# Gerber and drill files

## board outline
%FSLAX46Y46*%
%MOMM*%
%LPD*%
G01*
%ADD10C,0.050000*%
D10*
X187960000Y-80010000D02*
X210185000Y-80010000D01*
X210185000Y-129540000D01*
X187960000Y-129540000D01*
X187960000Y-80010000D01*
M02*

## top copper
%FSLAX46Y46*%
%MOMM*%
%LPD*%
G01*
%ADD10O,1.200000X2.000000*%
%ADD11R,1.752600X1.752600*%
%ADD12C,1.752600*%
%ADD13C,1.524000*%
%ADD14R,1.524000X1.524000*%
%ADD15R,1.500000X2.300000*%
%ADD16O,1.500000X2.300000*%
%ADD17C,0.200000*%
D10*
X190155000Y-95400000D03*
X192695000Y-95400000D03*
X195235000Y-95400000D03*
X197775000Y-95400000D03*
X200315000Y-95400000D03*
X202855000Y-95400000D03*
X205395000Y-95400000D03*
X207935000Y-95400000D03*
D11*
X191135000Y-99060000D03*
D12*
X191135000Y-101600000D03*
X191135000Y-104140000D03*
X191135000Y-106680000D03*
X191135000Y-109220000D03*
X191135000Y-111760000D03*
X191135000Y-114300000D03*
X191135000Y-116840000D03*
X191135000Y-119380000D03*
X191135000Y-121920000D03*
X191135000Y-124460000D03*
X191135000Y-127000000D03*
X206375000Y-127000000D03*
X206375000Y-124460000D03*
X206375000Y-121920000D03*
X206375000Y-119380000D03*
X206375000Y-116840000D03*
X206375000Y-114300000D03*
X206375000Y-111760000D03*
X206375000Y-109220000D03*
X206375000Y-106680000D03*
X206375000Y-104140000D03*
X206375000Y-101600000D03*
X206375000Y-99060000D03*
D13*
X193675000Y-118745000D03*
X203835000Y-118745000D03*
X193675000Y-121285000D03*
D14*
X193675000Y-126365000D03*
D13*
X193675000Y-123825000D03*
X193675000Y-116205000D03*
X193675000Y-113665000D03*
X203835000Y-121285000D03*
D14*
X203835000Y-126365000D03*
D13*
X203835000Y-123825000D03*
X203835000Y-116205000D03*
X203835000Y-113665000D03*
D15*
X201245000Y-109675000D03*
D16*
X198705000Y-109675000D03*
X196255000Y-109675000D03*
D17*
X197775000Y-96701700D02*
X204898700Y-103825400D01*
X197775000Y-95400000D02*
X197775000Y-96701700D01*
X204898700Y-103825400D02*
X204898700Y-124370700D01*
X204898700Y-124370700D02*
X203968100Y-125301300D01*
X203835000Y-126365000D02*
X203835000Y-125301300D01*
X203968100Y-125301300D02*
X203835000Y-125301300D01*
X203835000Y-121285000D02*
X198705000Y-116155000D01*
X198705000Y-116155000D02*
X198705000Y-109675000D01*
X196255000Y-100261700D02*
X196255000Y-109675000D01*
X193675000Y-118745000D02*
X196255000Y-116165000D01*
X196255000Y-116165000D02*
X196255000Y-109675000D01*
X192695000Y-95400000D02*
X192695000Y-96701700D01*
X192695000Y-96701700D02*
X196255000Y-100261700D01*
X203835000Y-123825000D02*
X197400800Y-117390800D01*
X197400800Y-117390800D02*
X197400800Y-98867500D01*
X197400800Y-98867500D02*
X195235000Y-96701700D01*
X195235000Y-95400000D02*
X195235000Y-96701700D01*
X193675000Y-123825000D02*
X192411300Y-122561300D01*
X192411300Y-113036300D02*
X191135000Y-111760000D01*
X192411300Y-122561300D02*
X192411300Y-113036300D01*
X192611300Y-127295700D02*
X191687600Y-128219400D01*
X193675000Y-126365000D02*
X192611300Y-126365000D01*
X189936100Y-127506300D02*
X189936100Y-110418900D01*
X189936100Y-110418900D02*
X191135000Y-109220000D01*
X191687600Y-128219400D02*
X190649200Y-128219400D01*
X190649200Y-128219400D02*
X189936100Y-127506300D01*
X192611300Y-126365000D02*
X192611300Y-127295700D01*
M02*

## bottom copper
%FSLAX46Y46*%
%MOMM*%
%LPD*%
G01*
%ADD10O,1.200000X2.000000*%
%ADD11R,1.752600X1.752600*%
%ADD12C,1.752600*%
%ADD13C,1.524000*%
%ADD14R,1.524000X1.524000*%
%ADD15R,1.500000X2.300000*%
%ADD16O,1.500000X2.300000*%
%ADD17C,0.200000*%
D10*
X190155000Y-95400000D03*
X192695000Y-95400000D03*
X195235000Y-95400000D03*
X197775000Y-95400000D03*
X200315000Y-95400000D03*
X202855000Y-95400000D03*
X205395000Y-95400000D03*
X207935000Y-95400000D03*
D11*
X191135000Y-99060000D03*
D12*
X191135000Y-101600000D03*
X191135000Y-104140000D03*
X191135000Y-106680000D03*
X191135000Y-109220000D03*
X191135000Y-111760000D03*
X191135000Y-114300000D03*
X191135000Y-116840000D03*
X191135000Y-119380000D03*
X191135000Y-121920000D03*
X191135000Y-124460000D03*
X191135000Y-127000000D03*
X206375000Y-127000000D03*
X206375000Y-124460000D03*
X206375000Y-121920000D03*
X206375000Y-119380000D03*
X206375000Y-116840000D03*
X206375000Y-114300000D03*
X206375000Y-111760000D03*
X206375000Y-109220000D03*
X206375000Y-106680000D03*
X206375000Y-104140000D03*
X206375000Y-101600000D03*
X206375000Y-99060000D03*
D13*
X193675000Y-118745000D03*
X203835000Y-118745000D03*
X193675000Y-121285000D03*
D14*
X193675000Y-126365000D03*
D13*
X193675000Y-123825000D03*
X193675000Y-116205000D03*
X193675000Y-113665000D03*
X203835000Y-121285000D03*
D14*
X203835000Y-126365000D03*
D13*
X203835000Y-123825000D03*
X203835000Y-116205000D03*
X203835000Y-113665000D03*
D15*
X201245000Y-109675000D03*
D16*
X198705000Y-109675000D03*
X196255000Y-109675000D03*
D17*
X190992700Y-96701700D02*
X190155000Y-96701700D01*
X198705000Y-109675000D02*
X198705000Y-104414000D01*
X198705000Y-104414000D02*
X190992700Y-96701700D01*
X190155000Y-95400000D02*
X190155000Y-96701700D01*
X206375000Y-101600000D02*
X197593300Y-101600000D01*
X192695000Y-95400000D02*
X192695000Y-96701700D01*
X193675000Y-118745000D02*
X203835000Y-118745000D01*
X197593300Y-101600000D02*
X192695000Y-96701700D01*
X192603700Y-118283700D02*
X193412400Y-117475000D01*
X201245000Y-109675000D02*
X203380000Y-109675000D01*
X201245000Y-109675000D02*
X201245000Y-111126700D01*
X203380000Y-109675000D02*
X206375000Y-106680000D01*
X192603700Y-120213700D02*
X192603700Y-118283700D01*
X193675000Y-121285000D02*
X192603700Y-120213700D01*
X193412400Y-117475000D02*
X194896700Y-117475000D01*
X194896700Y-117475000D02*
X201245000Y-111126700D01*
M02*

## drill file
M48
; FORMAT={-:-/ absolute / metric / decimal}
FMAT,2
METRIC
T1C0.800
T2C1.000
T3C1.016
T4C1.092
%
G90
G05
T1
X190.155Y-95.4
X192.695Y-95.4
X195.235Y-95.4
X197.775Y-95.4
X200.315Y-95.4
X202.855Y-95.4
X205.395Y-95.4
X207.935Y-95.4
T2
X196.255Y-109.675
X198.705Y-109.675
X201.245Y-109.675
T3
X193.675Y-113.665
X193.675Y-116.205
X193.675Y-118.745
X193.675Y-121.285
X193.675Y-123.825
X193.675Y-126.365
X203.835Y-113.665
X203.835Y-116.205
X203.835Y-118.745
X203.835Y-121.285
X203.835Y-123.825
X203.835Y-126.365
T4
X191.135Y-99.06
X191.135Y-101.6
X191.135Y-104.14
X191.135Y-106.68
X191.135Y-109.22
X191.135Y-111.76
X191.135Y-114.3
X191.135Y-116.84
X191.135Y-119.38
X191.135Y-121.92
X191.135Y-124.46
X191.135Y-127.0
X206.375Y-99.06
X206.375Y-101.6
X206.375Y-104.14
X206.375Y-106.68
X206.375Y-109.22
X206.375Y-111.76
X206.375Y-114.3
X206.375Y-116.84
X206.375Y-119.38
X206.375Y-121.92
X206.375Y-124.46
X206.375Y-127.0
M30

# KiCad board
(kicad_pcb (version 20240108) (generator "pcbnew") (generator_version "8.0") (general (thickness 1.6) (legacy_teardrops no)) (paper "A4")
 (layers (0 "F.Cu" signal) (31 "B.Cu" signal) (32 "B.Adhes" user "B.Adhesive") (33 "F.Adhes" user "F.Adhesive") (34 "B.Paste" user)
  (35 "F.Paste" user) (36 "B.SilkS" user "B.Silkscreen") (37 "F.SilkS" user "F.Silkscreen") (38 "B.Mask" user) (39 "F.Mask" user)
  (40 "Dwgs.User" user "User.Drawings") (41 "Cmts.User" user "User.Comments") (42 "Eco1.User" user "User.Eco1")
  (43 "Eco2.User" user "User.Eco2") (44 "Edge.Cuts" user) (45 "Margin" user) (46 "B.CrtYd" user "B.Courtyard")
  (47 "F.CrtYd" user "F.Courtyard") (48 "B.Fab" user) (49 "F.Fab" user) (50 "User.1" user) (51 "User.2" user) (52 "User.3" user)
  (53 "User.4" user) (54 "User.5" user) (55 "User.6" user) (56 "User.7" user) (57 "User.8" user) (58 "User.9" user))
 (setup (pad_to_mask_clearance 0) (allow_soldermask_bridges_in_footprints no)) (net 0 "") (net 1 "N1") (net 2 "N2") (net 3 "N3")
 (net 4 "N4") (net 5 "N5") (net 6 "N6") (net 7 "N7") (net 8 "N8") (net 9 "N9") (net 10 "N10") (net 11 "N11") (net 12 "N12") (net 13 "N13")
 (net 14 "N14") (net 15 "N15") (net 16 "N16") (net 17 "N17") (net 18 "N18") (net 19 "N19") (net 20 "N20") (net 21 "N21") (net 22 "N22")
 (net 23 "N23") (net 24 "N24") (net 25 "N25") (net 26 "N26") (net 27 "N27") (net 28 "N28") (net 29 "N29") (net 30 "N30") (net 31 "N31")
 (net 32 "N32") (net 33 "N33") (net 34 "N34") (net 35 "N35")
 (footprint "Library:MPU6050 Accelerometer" (layer "F.Cu") (at 201.295 88.9 90)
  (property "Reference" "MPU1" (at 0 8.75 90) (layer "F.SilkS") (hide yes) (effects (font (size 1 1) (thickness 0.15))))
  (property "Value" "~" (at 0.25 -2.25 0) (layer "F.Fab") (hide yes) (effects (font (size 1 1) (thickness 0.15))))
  (pad "1" thru_hole oval (at -6.5 -11.14) (size 1.2 2) (drill 0.8) (layers "*.Cu" "*.Mask") (remove_unused_layers no) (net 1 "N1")
   (thermal_bridge_angle 45))
  (pad "2" thru_hole oval (at -6.5 -8.6) (size 1.2 2) (drill 0.8) (layers "*.Cu" "*.Mask") (remove_unused_layers no) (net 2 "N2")
   (thermal_bridge_angle 45))
  (pad "3" thru_hole oval (at -6.5 -6.06) (size 1.2 2) (drill 0.8) (layers "*.Cu" "*.Mask") (remove_unused_layers no) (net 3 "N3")
   (thermal_bridge_angle 45))
  (pad "4" thru_hole oval (at -6.5 -3.52) (size 1.2 2) (drill 0.8) (layers "*.Cu" "*.Mask") (remove_unused_layers no) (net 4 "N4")
   (thermal_bridge_angle 45))
  (pad "5" thru_hole oval (at -6.5 -0.98) (size 1.2 2) (drill 0.8) (layers "*.Cu" "*.Mask") (remove_unused_layers no) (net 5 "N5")
   (thermal_bridge_angle 45))
  (pad "6" thru_hole oval (at -6.5 1.56) (size 1.2 2) (drill 0.8) (layers "*.Cu" "*.Mask") (remove_unused_layers no) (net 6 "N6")
   (thermal_bridge_angle 45))
  (pad "7" thru_hole oval (at -6.5 4.1) (size 1.2 2) (drill 0.8) (layers "*.Cu" "*.Mask") (remove_unused_layers no) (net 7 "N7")
   (thermal_bridge_angle 45))
  (pad "8" thru_hole oval (at -6.5 6.64) (size 1.2 2) (drill 0.8) (layers "*.Cu" "*.Mask") (remove_unused_layers no) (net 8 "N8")
   (thermal_bridge_angle 45)))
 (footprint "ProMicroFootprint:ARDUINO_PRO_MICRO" (layer "F.Cu") (at 198.755 113.03 -90)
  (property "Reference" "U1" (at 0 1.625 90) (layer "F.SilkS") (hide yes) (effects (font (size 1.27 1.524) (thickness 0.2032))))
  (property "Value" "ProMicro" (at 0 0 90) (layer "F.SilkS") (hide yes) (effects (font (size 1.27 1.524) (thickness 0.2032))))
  (pad "1" thru_hole rect (at -13.97 7.62 270) (size 1.7526 1.7526) (drill 1.0922) (layers "*.Cu" "*.SilkS" "*.Mask")
   (remove_unused_layers no) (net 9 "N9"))
  (pad "2" thru_hole circle (at -11.43 7.62 270) (size 1.7526 1.7526) (drill 1.0922) (layers "*.Cu" "*.SilkS" "*.Mask")
   (remove_unused_layers no) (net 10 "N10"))
  (pad "3" thru_hole circle (at -8.89 7.62 270) (size 1.7526 1.7526) (drill 1.0922) (layers "*.Cu" "*.SilkS" "*.Mask")
   (remove_unused_layers no) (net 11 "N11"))
  (pad "4" thru_hole circle (at -6.35 7.62 270) (size 1.7526 1.7526) (drill 1.0922) (layers "*.Cu" "*.SilkS" "*.Mask")
   (remove_unused_layers no) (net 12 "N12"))
  (pad "5" thru_hole circle (at -3.81 7.62 270) (size 1.7526 1.7526) (drill 1.0922) (layers "*.Cu" "*.SilkS" "*.Mask")
   (remove_unused_layers no) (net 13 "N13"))
  (pad "6" thru_hole circle (at -1.27 7.62 270) (size 1.7526 1.7526) (drill 1.0922) (layers "*.Cu" "*.SilkS" "*.Mask")
   (remove_unused_layers no) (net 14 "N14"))
  (pad "7" thru_hole circle (at 1.27 7.62 270) (size 1.7526 1.7526) (drill 1.0922) (layers "*.Cu" "*.SilkS" "*.Mask")
   (remove_unused_layers no) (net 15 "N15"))
  (pad "8" thru_hole circle (at 3.81 7.62 270) (size 1.7526 1.7526) (drill 1.0922) (layers "*.Cu" "*.SilkS" "*.Mask")
   (remove_unused_layers no) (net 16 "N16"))
  (pad "9" thru_hole circle (at 6.35 7.62 270) (size 1.7526 1.7526) (drill 1.0922) (layers "*.Cu" "*.SilkS" "*.Mask")
   (remove_unused_layers no) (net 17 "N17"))
  (pad "10" thru_hole circle (at 8.89 7.62 270) (size 1.7526 1.7526) (drill 1.0922) (layers "*.Cu" "*.SilkS" "*.Mask")
   (remove_unused_layers no) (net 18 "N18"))
  (pad "11" thru_hole circle (at 11.43 7.62 270) (size 1.7526 1.7526) (drill 1.0922) (layers "*.Cu" "*.SilkS" "*.Mask")
   (remove_unused_layers no) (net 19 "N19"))
  (pad "12" thru_hole circle (at 13.97 7.62 270) (size 1.7526 1.7526) (drill 1.0922) (layers "*.Cu" "*.SilkS" "*.Mask")
   (remove_unused_layers no) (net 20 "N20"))
  (pad "13" thru_hole circle (at 13.97 -7.62 270) (size 1.7526 1.7526) (drill 1.0922) (layers "*.Cu" "*.SilkS" "*.Mask")
   (remove_unused_layers no) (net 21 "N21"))
  (pad "14" thru_hole circle (at 11.43 -7.62 270) (size 1.7526 1.7526) (drill 1.0922) (layers "*.Cu" "*.SilkS" "*.Mask")
   (remove_unused_layers no) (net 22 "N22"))
  (pad "15" thru_hole circle (at 8.89 -7.62 270) (size 1.7526 1.7526) (drill 1.0922) (layers "*.Cu" "*.SilkS" "*.Mask")
   (remove_unused_layers no) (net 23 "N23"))
  (pad "16" thru_hole circle (at 6.35 -7.62 270) (size 1.7526 1.7526) (drill 1.0922) (layers "*.Cu" "*.SilkS" "*.Mask")
   (remove_unused_layers no) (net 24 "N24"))
  (pad "17" thru_hole circle (at 3.81 -7.62 270) (size 1.7526 1.7526) (drill 1.0922) (layers "*.Cu" "*.SilkS" "*.Mask")
   (remove_unused_layers no) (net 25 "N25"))
  (pad "18" thru_hole circle (at 1.27 -7.62 270) (size 1.7526 1.7526) (drill 1.0922) (layers "*.Cu" "*.SilkS" "*.Mask")
   (remove_unused_layers no) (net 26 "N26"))
  (pad "19" thru_hole circle (at -1.27 -7.62 270) (size 1.7526 1.7526) (drill 1.0922) (layers "*.Cu" "*.SilkS" "*.Mask")
   (remove_unused_layers no) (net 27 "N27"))
  (pad "20" thru_hole circle (at -3.81 -7.62 270) (size 1.7526 1.7526) (drill 1.0922) (layers "*.Cu" "*.SilkS" "*.Mask")
   (remove_unused_layers no) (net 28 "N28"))
  (pad "21" thru_hole circle (at -6.35 -7.62 270) (size 1.7526 1.7526) (drill 1.0922) (layers "*.Cu" "*.SilkS" "*.Mask")
   (remove_unused_layers no) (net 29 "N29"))
  (pad "22" thru_hole circle (at -8.89 -7.62 270) (size 1.7526 1.7526) (drill 1.0922) (layers "*.Cu" "*.SilkS" "*.Mask")
   (remove_unused_layers no) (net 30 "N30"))
  (pad "23" thru_hole circle (at -11.43 -7.62 270) (size 1.7526 1.7526) (drill 1.0922) (layers "*.Cu" "*.SilkS" "*.Mask")
   (remove_unused_layers no) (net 2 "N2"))
  (pad "24" thru_hole circle (at -13.97 -7.62 270) (size 1.7526 1.7526) (drill 1.0922) (layers "*.Cu" "*.SilkS" "*.Mask")
   (remove_unused_layers no) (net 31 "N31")))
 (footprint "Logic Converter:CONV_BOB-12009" (layer "F.Cu") (at 198.755 120.015 180)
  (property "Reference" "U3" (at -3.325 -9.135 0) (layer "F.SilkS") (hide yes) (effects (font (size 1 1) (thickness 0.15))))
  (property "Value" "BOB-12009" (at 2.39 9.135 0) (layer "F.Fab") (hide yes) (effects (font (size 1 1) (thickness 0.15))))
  (pad "GND_1" thru_hole circle (at 5.08 1.27 180) (size 1.524 1.524) (drill 1.016) (layers "*.Cu" "*.Mask") (remove_unused_layers no)
   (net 2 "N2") (solder_mask_margin 0.102))
  (pad "GND_2" thru_hole circle (at -5.08 1.27 180) (size 1.524 1.524) (drill 1.016) (layers "*.Cu" "*.Mask") (remove_unused_layers no)
   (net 2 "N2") (solder_mask_margin 0.102))
  (pad "HV" thru_hole circle (at 5.08 -1.27 180) (size 1.524 1.524) (drill 1.016) (layers "*.Cu" "*.Mask") (remove_unused_layers no)
   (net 29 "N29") (solder_mask_margin 0.102))
  (pad "HV1" thru_hole rect (at 5.08 -6.35 180) (size 1.524 1.524) (drill 1.016) (layers "*.Cu" "*.Mask") (remove_unused_layers no)
   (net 13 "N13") (solder_mask_margin 0.102))
  (pad "HV2" thru_hole circle (at 5.08 -3.81 180) (size 1.524 1.524) (drill 1.016) (layers "*.Cu" "*.Mask") (remove_unused_layers no)
   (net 14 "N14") (solder_mask_margin 0.102))
  (pad "HV3" thru_hole circle (at 5.08 3.81 180) (size 1.524 1.524) (drill 1.016) (layers "*.Cu" "*.Mask") (remove_unused_layers no)
   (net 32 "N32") (solder_mask_margin 0.102))
  (pad "HV4" thru_hole circle (at 5.08 6.35 180) (size 1.524 1.524) (drill 1.016) (layers "*.Cu" "*.Mask") (remove_unused_layers no)
   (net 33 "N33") (solder_mask_margin 0.102))
  (pad "LV" thru_hole circle (at -5.08 -1.27 180) (size 1.524 1.524) (drill 1.016) (layers "*.Cu" "*.Mask") (remove_unused_layers no)
   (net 1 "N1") (solder_mask_margin 0.102))
  (pad "LV1" thru_hole rect (at -5.08 -6.35 180) (size 1.524 1.524) (drill 1.016) (layers "*.Cu" "*.Mask") (remove_unused_layers no)
   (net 4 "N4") (solder_mask_margin 0.102))
  (pad "LV2" thru_hole circle (at -5.08 -3.81 180) (size 1.524 1.524) (drill 1.016) (layers "*.Cu" "*.Mask") (remove_unused_layers no)
   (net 3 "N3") (solder_mask_margin 0.102))
  (pad "LV3" thru_hole circle (at -5.08 3.81 180) (size 1.524 1.524) (drill 1.016) (layers "*.Cu" "*.Mask") (remove_unused_layers no)
   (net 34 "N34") (solder_mask_margin 0.102))
  (pad "LV4" thru_hole circle (at -5.08 6.35 180) (size 1.524 1.524) (drill 1.016) (layers "*.Cu" "*.Mask") (remove_unused_layers no)
   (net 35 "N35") (solder_mask_margin 0.102)))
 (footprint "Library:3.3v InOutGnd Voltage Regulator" (layer "F.Cu") (at 198.755 111.175)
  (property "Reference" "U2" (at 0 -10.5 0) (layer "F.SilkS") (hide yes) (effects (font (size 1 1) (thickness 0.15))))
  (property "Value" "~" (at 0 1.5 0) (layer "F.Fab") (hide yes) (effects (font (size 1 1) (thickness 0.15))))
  (pad "1" thru_hole rect (at 2.49 -1.5) (size 1.5 2.3) (drill 1) (layers "*.Cu" "*.Mask") (remove_unused_layers no) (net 29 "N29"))
  (pad "2" thru_hole oval (at -0.05 -1.5) (size 1.5 2.3) (drill 1) (layers "*.Cu" "*.Mask") (remove_unused_layers no) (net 1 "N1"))
  (pad "3" thru_hole oval (at -2.5 -1.5) (size 1.5 2.3) (drill 1) (layers "*.Cu" "*.Mask") (remove_unused_layers no) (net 2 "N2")))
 (gr_rect (start 187.96 80.01) (end 210.185 129.54) (stroke (width 0.05) (type default)) (fill none) (layer "Edge.Cuts"))
 (segment (start 197.775 96.7017) (end 204.8987 103.8254) (width 0.2) (layer "F.Cu") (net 4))
 (segment (start 197.775 95.4) (end 197.775 96.7017) (width 0.2) (layer "F.Cu") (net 4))
 (segment (start 204.8987 103.8254) (end 204.8987 124.3707) (width 0.2) (layer "F.Cu") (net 4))
 (segment (start 204.8987 124.3707) (end 203.9681 125.3013) (width 0.2) (layer "F.Cu") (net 4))
 (segment (start 203.835 126.365) (end 203.835 125.3013) (width 0.2) (layer "F.Cu") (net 4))
 (segment (start 203.9681 125.3013) (end 203.835 125.3013) (width 0.2) (layer "F.Cu") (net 4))
 (segment (start 203.835 121.285) (end 198.705 116.155) (width 0.2) (layer "F.Cu") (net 1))
 (segment (start 198.705 116.155) (end 198.705 109.675) (width 0.2) (layer "F.Cu") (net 1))
 (segment (start 190.9927 96.7017) (end 190.155 96.7017) (width 0.2) (layer "B.Cu") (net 1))
 (segment (start 198.705 109.675) (end 198.705 104.414) (width 0.2) (layer "B.Cu") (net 1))
 (segment (start 198.705 104.414) (end 190.9927 96.7017) (width 0.2) (layer "B.Cu") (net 1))
 (segment (start 190.155 95.4) (end 190.155 96.7017) (width 0.2) (layer "B.Cu") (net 1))
 (segment (start 196.255 100.2617) (end 196.255 109.675) (width 0.2) (layer "F.Cu") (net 2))
 (segment (start 193.675 118.745) (end 196.255 116.165) (width 0.2) (layer "F.Cu") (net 2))
 (segment (start 196.255 116.165) (end 196.255 109.675) (width 0.2) (layer "F.Cu") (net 2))
 (segment (start 192.695 95.4) (end 192.695 96.7017) (width 0.2) (layer "F.Cu") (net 2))
 (segment (start 192.695 96.7017) (end 196.255 100.2617) (width 0.2) (layer "F.Cu") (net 2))
 (segment (start 206.375 101.6) (end 197.5933 101.6) (width 0.2) (layer "B.Cu") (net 2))
 (segment (start 192.695 95.4) (end 192.695 96.7017) (width 0.2) (layer "B.Cu") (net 2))
 (segment (start 193.675 118.745) (end 203.835 118.745) (width 0.2) (layer "B.Cu") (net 2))
 (segment (start 197.5933 101.6) (end 192.695 96.7017) (width 0.2) (layer "B.Cu") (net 2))
 (segment (start 203.835 123.825) (end 197.4008 117.3908) (width 0.2) (layer "F.Cu") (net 3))
 (segment (start 197.4008 117.3908) (end 197.4008 98.8675) (width 0.2) (layer "F.Cu") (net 3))
 (segment (start 197.4008 98.8675) (end 195.235 96.7017) (width 0.2) (layer "F.Cu") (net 3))
 (segment (start 195.235 95.4) (end 195.235 96.7017) (width 0.2) (layer "F.Cu") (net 3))
 (segment (start 192.6037 118.2837) (end 193.4124 117.475) (width 0.2) (layer "B.Cu") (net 29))
 (segment (start 201.245 109.675) (end 203.38 109.675) (width 0.2) (layer "B.Cu") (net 29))
 (segment (start 201.245 109.675) (end 201.245 111.1267) (width 0.2) (layer "B.Cu") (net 29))
 (segment (start 203.38 109.675) (end 206.375 106.68) (width 0.2) (layer "B.Cu") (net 29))
 (segment (start 192.6037 120.2137) (end 192.6037 118.2837) (width 0.2) (layer "B.Cu") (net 29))
 (segment (start 193.675 121.285) (end 192.6037 120.2137) (width 0.2) (layer "B.Cu") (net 29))
 (segment (start 193.4124 117.475) (end 194.8967 117.475) (width 0.2) (layer "B.Cu") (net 29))
 (segment (start 194.8967 117.475) (end 201.245 111.1267) (width 0.2) (layer "B.Cu") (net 29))
 (segment (start 193.675 123.825) (end 192.4113 122.5613) (width 0.2) (layer "F.Cu") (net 14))
 (segment (start 192.4113 113.0363) (end 191.135 111.76) (width 0.2) (layer "F.Cu") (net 14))
 (segment (start 192.4113 122.5613) (end 192.4113 113.0363) (width 0.2) (layer "F.Cu") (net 14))
 (segment (start 192.6113 127.2957) (end 191.6876 128.2194) (width 0.2) (layer "F.Cu") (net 13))
 (segment (start 193.675 126.365) (end 192.6113 126.365) (width 0.2) (layer "F.Cu") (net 13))
 (segment (start 189.9361 127.5063) (end 189.9361 110.4189) (width 0.2) (layer "F.Cu") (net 13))
 (segment (start 189.9361 110.4189) (end 191.135 109.22) (width 0.2) (layer "F.Cu") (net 13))
 (segment (start 191.6876 128.2194) (end 190.6492 128.2194) (width 0.2) (layer "F.Cu") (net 13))
 (segment (start 190.6492 128.2194) (end 189.9361 127.5063) (width 0.2) (layer "F.Cu") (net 13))
 (segment (start 192.6113 126.365) (end 192.6113 127.2957) (width 0.2) (layer "F.Cu") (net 13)))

